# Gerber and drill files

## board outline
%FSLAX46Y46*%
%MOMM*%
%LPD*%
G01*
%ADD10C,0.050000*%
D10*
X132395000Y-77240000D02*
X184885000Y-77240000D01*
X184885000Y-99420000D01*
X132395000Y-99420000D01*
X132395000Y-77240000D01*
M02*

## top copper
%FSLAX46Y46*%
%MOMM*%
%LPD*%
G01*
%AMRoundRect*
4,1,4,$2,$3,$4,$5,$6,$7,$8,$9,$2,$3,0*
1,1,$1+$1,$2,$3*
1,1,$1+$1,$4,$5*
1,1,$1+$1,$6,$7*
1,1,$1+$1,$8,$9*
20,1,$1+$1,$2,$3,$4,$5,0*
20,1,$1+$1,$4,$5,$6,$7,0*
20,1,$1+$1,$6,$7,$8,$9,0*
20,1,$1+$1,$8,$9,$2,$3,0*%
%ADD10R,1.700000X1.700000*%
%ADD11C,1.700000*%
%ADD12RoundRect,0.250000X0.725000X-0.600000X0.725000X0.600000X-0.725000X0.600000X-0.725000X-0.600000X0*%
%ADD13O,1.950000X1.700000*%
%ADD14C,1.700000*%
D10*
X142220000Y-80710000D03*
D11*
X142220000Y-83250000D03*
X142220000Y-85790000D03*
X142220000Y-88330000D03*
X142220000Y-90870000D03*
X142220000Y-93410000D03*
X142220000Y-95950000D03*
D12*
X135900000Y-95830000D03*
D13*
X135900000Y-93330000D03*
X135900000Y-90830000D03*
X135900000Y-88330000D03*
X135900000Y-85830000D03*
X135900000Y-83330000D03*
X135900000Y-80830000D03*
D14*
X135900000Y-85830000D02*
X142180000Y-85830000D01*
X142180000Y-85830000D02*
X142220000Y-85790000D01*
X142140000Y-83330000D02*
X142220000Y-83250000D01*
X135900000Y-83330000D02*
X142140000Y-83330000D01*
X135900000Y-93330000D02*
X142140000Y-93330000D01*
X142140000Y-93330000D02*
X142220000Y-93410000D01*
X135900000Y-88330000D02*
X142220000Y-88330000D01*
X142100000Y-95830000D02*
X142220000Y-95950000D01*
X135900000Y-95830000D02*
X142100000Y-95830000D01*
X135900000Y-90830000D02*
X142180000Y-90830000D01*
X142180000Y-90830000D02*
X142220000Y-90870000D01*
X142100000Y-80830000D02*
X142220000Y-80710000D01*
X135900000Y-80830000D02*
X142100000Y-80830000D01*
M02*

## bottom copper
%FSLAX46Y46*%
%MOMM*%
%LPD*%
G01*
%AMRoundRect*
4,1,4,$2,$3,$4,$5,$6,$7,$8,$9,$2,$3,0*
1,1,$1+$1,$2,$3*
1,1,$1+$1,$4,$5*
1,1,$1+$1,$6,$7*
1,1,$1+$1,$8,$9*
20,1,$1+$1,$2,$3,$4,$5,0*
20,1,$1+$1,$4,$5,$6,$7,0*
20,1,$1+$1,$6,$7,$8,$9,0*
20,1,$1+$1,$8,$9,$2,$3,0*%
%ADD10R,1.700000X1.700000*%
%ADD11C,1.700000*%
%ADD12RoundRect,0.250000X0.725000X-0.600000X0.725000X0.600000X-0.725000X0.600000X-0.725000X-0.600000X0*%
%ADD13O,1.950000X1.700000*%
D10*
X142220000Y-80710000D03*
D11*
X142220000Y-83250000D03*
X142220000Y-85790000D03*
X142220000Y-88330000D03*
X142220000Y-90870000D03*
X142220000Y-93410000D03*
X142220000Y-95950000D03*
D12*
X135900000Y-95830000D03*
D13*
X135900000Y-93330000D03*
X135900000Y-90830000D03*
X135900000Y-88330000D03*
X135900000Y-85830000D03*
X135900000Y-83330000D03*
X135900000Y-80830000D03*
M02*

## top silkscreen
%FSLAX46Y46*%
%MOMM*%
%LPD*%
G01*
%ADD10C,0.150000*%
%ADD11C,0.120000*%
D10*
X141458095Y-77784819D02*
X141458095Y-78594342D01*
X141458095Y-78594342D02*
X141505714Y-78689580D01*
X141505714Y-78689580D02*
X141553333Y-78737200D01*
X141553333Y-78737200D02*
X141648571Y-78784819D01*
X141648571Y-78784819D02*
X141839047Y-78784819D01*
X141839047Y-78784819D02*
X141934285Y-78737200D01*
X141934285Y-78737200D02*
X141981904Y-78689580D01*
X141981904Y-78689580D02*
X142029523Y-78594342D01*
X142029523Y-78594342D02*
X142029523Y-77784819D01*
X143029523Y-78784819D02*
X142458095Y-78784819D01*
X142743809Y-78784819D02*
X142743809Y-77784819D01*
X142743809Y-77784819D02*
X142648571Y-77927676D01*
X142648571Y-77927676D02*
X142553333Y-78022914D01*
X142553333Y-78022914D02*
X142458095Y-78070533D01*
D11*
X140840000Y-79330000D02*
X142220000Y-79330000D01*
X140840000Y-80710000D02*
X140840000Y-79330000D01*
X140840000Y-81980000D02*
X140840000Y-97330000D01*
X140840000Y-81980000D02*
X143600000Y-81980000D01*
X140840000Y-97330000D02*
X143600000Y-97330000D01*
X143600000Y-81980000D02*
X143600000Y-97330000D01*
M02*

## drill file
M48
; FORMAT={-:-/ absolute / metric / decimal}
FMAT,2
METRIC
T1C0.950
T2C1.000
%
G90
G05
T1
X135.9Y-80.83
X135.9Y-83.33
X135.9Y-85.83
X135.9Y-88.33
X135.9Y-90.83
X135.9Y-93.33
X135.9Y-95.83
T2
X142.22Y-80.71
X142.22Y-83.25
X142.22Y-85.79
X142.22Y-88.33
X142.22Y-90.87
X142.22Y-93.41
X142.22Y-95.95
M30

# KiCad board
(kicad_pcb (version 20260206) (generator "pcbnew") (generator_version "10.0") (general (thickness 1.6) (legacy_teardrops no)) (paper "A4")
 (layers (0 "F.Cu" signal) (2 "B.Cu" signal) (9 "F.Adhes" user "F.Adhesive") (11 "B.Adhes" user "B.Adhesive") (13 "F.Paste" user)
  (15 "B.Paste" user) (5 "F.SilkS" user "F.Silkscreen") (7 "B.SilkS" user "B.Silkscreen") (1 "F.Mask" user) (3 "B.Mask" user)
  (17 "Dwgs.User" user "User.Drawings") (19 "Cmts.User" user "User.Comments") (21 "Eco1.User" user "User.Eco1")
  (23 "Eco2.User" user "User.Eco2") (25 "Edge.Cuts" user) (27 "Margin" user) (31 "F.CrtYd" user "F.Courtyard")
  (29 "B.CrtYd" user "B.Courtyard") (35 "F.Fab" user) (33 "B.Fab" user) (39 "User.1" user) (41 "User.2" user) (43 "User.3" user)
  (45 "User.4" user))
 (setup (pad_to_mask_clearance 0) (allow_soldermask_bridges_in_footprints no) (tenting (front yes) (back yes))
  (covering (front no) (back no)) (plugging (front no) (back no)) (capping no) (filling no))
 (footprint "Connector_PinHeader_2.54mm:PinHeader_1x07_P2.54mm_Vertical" (layer "F.Cu") (at 142.22 80.71)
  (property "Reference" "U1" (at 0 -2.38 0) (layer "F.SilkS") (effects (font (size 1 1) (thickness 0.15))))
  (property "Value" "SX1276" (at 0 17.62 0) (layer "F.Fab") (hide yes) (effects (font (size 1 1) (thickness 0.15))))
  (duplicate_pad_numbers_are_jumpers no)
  (fp_line (start -1.38 -1.38) (end 0 -1.38) (stroke (width 0.12) (type solid)) (layer "F.SilkS"))
  (fp_line (start -1.38 0) (end -1.38 -1.38) (stroke (width 0.12) (type solid)) (layer "F.SilkS"))
  (fp_line (start -1.38 1.27) (end -1.38 16.62) (stroke (width 0.12) (type solid)) (layer "F.SilkS"))
  (fp_line (start -1.38 1.27) (end 1.38 1.27) (stroke (width 0.12) (type solid)) (layer "F.SilkS"))
  (fp_line (start -1.38 16.62) (end 1.38 16.62) (stroke (width 0.12) (type solid)) (layer "F.SilkS"))
  (fp_line (start 1.38 1.27) (end 1.38 16.62) (stroke (width 0.12) (type solid)) (layer "F.SilkS"))
  (pad "1" thru_hole rect (at 0 0) (size 1.7 1.7) (drill 1) (layers "*.Cu" "*.Mask") (remove_unused_layers no) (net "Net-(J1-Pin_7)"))
  (pad "2" thru_hole circle (at 0 2.54) (size 1.7 1.7) (drill 1) (layers "*.Cu" "*.Mask") (remove_unused_layers no) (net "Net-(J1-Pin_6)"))
  (pad "3" thru_hole circle (at 0 5.08) (size 1.7 1.7) (drill 1) (layers "*.Cu" "*.Mask") (remove_unused_layers no) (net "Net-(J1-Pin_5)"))
  (pad "4" thru_hole circle (at 0 7.62) (size 1.7 1.7) (drill 1) (layers "*.Cu" "*.Mask") (remove_unused_layers no) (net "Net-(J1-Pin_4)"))
  (pad "5" thru_hole circle (at 0 10.16) (size 1.7 1.7) (drill 1) (layers "*.Cu" "*.Mask") (remove_unused_layers no) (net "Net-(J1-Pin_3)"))
  (pad "6" thru_hole circle (at 0 12.7) (size 1.7 1.7) (drill 1) (layers "*.Cu" "*.Mask") (remove_unused_layers no) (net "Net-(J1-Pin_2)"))
  (pad "7" thru_hole circle (at 0 15.24) (size 1.7 1.7) (drill 1) (layers "*.Cu" "*.Mask") (remove_unused_layers no) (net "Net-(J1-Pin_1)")))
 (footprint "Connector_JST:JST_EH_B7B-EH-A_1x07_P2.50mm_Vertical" (layer "B.Cu") (at 135.9 95.83 90)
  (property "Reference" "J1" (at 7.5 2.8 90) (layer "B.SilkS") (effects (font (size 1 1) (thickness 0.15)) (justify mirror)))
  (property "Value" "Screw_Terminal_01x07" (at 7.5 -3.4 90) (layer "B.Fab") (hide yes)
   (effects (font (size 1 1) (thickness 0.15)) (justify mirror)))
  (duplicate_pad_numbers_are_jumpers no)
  (pad "1" thru_hole roundrect (at 0 0 90) (size 1.7 1.95) (drill 0.95) (layers "*.Cu" "*.Mask") (remove_unused_layers no)
   (roundrect_rratio 0.147059) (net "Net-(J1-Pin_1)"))
  (pad "2" thru_hole oval (at 2.5 0 90) (size 1.7 1.95) (drill 0.95) (layers "*.Cu" "*.Mask") (remove_unused_layers no)
   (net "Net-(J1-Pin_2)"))
  (pad "3" thru_hole oval (at 5 0 90) (size 1.7 1.95) (drill 0.95) (layers "*.Cu" "*.Mask") (remove_unused_layers no) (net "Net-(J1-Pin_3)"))
  (pad "4" thru_hole oval (at 7.5 0 90) (size 1.7 1.95) (drill 0.95) (layers "*.Cu" "*.Mask") (remove_unused_layers no)
   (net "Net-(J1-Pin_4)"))
  (pad "5" thru_hole oval (at 10 0 90) (size 1.7 1.95) (drill 0.95) (layers "*.Cu" "*.Mask") (remove_unused_layers no)
   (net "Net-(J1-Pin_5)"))
  (pad "6" thru_hole oval (at 12.5 0 90) (size 1.7 1.95) (drill 0.95) (layers "*.Cu" "*.Mask") (remove_unused_layers no)
   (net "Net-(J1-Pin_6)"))
  (pad "7" thru_hole oval (at 15 0 90) (size 1.7 1.95) (drill 0.95) (layers "*.Cu" "*.Mask") (remove_unused_layers no)
   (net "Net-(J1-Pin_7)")))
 (gr_rect (start 132.395 77.24) (end 184.885 99.42) (stroke (width 0.05) (type default)) (fill no) (layer "Edge.Cuts"))
 (segment (start 135.9 85.83) (end 142.18 85.83) (width 1.7) (layer "F.Cu") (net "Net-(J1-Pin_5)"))
 (segment (start 142.18 85.83) (end 142.22 85.79) (width 1.7) (layer "F.Cu") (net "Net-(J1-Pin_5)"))
 (segment (start 142.14 83.33) (end 142.22 83.25) (width 1.7) (layer "F.Cu") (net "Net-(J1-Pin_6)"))
 (segment (start 135.9 83.33) (end 142.14 83.33) (width 1.7) (layer "F.Cu") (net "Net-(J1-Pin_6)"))
 (segment (start 135.9 93.33) (end 142.14 93.33) (width 1.7) (layer "F.Cu") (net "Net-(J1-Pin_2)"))
 (segment (start 142.14 93.33) (end 142.22 93.41) (width 1.7) (layer "F.Cu") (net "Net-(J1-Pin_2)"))
 (segment (start 135.9 88.33) (end 142.22 88.33) (width 1.7) (layer "F.Cu") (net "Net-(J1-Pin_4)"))
 (segment (start 142.1 95.83) (end 142.22 95.95) (width 1.7) (layer "F.Cu") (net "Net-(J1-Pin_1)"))
 (segment (start 135.9 95.83) (end 142.1 95.83) (width 1.7) (layer "F.Cu") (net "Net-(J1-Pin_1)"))
 (segment (start 135.9 90.83) (end 142.18 90.83) (width 1.7) (layer "F.Cu") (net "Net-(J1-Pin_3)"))
 (segment (start 142.18 90.83) (end 142.22 90.87) (width 1.7) (layer "F.Cu") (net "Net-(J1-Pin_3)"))
 (segment (start 142.1 80.83) (end 142.22 80.71) (width 1.7) (layer "F.Cu") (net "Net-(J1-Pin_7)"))
 (segment (start 135.9 80.83) (end 142.1 80.83) (width 1.7) (layer "F.Cu") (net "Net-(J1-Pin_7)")))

